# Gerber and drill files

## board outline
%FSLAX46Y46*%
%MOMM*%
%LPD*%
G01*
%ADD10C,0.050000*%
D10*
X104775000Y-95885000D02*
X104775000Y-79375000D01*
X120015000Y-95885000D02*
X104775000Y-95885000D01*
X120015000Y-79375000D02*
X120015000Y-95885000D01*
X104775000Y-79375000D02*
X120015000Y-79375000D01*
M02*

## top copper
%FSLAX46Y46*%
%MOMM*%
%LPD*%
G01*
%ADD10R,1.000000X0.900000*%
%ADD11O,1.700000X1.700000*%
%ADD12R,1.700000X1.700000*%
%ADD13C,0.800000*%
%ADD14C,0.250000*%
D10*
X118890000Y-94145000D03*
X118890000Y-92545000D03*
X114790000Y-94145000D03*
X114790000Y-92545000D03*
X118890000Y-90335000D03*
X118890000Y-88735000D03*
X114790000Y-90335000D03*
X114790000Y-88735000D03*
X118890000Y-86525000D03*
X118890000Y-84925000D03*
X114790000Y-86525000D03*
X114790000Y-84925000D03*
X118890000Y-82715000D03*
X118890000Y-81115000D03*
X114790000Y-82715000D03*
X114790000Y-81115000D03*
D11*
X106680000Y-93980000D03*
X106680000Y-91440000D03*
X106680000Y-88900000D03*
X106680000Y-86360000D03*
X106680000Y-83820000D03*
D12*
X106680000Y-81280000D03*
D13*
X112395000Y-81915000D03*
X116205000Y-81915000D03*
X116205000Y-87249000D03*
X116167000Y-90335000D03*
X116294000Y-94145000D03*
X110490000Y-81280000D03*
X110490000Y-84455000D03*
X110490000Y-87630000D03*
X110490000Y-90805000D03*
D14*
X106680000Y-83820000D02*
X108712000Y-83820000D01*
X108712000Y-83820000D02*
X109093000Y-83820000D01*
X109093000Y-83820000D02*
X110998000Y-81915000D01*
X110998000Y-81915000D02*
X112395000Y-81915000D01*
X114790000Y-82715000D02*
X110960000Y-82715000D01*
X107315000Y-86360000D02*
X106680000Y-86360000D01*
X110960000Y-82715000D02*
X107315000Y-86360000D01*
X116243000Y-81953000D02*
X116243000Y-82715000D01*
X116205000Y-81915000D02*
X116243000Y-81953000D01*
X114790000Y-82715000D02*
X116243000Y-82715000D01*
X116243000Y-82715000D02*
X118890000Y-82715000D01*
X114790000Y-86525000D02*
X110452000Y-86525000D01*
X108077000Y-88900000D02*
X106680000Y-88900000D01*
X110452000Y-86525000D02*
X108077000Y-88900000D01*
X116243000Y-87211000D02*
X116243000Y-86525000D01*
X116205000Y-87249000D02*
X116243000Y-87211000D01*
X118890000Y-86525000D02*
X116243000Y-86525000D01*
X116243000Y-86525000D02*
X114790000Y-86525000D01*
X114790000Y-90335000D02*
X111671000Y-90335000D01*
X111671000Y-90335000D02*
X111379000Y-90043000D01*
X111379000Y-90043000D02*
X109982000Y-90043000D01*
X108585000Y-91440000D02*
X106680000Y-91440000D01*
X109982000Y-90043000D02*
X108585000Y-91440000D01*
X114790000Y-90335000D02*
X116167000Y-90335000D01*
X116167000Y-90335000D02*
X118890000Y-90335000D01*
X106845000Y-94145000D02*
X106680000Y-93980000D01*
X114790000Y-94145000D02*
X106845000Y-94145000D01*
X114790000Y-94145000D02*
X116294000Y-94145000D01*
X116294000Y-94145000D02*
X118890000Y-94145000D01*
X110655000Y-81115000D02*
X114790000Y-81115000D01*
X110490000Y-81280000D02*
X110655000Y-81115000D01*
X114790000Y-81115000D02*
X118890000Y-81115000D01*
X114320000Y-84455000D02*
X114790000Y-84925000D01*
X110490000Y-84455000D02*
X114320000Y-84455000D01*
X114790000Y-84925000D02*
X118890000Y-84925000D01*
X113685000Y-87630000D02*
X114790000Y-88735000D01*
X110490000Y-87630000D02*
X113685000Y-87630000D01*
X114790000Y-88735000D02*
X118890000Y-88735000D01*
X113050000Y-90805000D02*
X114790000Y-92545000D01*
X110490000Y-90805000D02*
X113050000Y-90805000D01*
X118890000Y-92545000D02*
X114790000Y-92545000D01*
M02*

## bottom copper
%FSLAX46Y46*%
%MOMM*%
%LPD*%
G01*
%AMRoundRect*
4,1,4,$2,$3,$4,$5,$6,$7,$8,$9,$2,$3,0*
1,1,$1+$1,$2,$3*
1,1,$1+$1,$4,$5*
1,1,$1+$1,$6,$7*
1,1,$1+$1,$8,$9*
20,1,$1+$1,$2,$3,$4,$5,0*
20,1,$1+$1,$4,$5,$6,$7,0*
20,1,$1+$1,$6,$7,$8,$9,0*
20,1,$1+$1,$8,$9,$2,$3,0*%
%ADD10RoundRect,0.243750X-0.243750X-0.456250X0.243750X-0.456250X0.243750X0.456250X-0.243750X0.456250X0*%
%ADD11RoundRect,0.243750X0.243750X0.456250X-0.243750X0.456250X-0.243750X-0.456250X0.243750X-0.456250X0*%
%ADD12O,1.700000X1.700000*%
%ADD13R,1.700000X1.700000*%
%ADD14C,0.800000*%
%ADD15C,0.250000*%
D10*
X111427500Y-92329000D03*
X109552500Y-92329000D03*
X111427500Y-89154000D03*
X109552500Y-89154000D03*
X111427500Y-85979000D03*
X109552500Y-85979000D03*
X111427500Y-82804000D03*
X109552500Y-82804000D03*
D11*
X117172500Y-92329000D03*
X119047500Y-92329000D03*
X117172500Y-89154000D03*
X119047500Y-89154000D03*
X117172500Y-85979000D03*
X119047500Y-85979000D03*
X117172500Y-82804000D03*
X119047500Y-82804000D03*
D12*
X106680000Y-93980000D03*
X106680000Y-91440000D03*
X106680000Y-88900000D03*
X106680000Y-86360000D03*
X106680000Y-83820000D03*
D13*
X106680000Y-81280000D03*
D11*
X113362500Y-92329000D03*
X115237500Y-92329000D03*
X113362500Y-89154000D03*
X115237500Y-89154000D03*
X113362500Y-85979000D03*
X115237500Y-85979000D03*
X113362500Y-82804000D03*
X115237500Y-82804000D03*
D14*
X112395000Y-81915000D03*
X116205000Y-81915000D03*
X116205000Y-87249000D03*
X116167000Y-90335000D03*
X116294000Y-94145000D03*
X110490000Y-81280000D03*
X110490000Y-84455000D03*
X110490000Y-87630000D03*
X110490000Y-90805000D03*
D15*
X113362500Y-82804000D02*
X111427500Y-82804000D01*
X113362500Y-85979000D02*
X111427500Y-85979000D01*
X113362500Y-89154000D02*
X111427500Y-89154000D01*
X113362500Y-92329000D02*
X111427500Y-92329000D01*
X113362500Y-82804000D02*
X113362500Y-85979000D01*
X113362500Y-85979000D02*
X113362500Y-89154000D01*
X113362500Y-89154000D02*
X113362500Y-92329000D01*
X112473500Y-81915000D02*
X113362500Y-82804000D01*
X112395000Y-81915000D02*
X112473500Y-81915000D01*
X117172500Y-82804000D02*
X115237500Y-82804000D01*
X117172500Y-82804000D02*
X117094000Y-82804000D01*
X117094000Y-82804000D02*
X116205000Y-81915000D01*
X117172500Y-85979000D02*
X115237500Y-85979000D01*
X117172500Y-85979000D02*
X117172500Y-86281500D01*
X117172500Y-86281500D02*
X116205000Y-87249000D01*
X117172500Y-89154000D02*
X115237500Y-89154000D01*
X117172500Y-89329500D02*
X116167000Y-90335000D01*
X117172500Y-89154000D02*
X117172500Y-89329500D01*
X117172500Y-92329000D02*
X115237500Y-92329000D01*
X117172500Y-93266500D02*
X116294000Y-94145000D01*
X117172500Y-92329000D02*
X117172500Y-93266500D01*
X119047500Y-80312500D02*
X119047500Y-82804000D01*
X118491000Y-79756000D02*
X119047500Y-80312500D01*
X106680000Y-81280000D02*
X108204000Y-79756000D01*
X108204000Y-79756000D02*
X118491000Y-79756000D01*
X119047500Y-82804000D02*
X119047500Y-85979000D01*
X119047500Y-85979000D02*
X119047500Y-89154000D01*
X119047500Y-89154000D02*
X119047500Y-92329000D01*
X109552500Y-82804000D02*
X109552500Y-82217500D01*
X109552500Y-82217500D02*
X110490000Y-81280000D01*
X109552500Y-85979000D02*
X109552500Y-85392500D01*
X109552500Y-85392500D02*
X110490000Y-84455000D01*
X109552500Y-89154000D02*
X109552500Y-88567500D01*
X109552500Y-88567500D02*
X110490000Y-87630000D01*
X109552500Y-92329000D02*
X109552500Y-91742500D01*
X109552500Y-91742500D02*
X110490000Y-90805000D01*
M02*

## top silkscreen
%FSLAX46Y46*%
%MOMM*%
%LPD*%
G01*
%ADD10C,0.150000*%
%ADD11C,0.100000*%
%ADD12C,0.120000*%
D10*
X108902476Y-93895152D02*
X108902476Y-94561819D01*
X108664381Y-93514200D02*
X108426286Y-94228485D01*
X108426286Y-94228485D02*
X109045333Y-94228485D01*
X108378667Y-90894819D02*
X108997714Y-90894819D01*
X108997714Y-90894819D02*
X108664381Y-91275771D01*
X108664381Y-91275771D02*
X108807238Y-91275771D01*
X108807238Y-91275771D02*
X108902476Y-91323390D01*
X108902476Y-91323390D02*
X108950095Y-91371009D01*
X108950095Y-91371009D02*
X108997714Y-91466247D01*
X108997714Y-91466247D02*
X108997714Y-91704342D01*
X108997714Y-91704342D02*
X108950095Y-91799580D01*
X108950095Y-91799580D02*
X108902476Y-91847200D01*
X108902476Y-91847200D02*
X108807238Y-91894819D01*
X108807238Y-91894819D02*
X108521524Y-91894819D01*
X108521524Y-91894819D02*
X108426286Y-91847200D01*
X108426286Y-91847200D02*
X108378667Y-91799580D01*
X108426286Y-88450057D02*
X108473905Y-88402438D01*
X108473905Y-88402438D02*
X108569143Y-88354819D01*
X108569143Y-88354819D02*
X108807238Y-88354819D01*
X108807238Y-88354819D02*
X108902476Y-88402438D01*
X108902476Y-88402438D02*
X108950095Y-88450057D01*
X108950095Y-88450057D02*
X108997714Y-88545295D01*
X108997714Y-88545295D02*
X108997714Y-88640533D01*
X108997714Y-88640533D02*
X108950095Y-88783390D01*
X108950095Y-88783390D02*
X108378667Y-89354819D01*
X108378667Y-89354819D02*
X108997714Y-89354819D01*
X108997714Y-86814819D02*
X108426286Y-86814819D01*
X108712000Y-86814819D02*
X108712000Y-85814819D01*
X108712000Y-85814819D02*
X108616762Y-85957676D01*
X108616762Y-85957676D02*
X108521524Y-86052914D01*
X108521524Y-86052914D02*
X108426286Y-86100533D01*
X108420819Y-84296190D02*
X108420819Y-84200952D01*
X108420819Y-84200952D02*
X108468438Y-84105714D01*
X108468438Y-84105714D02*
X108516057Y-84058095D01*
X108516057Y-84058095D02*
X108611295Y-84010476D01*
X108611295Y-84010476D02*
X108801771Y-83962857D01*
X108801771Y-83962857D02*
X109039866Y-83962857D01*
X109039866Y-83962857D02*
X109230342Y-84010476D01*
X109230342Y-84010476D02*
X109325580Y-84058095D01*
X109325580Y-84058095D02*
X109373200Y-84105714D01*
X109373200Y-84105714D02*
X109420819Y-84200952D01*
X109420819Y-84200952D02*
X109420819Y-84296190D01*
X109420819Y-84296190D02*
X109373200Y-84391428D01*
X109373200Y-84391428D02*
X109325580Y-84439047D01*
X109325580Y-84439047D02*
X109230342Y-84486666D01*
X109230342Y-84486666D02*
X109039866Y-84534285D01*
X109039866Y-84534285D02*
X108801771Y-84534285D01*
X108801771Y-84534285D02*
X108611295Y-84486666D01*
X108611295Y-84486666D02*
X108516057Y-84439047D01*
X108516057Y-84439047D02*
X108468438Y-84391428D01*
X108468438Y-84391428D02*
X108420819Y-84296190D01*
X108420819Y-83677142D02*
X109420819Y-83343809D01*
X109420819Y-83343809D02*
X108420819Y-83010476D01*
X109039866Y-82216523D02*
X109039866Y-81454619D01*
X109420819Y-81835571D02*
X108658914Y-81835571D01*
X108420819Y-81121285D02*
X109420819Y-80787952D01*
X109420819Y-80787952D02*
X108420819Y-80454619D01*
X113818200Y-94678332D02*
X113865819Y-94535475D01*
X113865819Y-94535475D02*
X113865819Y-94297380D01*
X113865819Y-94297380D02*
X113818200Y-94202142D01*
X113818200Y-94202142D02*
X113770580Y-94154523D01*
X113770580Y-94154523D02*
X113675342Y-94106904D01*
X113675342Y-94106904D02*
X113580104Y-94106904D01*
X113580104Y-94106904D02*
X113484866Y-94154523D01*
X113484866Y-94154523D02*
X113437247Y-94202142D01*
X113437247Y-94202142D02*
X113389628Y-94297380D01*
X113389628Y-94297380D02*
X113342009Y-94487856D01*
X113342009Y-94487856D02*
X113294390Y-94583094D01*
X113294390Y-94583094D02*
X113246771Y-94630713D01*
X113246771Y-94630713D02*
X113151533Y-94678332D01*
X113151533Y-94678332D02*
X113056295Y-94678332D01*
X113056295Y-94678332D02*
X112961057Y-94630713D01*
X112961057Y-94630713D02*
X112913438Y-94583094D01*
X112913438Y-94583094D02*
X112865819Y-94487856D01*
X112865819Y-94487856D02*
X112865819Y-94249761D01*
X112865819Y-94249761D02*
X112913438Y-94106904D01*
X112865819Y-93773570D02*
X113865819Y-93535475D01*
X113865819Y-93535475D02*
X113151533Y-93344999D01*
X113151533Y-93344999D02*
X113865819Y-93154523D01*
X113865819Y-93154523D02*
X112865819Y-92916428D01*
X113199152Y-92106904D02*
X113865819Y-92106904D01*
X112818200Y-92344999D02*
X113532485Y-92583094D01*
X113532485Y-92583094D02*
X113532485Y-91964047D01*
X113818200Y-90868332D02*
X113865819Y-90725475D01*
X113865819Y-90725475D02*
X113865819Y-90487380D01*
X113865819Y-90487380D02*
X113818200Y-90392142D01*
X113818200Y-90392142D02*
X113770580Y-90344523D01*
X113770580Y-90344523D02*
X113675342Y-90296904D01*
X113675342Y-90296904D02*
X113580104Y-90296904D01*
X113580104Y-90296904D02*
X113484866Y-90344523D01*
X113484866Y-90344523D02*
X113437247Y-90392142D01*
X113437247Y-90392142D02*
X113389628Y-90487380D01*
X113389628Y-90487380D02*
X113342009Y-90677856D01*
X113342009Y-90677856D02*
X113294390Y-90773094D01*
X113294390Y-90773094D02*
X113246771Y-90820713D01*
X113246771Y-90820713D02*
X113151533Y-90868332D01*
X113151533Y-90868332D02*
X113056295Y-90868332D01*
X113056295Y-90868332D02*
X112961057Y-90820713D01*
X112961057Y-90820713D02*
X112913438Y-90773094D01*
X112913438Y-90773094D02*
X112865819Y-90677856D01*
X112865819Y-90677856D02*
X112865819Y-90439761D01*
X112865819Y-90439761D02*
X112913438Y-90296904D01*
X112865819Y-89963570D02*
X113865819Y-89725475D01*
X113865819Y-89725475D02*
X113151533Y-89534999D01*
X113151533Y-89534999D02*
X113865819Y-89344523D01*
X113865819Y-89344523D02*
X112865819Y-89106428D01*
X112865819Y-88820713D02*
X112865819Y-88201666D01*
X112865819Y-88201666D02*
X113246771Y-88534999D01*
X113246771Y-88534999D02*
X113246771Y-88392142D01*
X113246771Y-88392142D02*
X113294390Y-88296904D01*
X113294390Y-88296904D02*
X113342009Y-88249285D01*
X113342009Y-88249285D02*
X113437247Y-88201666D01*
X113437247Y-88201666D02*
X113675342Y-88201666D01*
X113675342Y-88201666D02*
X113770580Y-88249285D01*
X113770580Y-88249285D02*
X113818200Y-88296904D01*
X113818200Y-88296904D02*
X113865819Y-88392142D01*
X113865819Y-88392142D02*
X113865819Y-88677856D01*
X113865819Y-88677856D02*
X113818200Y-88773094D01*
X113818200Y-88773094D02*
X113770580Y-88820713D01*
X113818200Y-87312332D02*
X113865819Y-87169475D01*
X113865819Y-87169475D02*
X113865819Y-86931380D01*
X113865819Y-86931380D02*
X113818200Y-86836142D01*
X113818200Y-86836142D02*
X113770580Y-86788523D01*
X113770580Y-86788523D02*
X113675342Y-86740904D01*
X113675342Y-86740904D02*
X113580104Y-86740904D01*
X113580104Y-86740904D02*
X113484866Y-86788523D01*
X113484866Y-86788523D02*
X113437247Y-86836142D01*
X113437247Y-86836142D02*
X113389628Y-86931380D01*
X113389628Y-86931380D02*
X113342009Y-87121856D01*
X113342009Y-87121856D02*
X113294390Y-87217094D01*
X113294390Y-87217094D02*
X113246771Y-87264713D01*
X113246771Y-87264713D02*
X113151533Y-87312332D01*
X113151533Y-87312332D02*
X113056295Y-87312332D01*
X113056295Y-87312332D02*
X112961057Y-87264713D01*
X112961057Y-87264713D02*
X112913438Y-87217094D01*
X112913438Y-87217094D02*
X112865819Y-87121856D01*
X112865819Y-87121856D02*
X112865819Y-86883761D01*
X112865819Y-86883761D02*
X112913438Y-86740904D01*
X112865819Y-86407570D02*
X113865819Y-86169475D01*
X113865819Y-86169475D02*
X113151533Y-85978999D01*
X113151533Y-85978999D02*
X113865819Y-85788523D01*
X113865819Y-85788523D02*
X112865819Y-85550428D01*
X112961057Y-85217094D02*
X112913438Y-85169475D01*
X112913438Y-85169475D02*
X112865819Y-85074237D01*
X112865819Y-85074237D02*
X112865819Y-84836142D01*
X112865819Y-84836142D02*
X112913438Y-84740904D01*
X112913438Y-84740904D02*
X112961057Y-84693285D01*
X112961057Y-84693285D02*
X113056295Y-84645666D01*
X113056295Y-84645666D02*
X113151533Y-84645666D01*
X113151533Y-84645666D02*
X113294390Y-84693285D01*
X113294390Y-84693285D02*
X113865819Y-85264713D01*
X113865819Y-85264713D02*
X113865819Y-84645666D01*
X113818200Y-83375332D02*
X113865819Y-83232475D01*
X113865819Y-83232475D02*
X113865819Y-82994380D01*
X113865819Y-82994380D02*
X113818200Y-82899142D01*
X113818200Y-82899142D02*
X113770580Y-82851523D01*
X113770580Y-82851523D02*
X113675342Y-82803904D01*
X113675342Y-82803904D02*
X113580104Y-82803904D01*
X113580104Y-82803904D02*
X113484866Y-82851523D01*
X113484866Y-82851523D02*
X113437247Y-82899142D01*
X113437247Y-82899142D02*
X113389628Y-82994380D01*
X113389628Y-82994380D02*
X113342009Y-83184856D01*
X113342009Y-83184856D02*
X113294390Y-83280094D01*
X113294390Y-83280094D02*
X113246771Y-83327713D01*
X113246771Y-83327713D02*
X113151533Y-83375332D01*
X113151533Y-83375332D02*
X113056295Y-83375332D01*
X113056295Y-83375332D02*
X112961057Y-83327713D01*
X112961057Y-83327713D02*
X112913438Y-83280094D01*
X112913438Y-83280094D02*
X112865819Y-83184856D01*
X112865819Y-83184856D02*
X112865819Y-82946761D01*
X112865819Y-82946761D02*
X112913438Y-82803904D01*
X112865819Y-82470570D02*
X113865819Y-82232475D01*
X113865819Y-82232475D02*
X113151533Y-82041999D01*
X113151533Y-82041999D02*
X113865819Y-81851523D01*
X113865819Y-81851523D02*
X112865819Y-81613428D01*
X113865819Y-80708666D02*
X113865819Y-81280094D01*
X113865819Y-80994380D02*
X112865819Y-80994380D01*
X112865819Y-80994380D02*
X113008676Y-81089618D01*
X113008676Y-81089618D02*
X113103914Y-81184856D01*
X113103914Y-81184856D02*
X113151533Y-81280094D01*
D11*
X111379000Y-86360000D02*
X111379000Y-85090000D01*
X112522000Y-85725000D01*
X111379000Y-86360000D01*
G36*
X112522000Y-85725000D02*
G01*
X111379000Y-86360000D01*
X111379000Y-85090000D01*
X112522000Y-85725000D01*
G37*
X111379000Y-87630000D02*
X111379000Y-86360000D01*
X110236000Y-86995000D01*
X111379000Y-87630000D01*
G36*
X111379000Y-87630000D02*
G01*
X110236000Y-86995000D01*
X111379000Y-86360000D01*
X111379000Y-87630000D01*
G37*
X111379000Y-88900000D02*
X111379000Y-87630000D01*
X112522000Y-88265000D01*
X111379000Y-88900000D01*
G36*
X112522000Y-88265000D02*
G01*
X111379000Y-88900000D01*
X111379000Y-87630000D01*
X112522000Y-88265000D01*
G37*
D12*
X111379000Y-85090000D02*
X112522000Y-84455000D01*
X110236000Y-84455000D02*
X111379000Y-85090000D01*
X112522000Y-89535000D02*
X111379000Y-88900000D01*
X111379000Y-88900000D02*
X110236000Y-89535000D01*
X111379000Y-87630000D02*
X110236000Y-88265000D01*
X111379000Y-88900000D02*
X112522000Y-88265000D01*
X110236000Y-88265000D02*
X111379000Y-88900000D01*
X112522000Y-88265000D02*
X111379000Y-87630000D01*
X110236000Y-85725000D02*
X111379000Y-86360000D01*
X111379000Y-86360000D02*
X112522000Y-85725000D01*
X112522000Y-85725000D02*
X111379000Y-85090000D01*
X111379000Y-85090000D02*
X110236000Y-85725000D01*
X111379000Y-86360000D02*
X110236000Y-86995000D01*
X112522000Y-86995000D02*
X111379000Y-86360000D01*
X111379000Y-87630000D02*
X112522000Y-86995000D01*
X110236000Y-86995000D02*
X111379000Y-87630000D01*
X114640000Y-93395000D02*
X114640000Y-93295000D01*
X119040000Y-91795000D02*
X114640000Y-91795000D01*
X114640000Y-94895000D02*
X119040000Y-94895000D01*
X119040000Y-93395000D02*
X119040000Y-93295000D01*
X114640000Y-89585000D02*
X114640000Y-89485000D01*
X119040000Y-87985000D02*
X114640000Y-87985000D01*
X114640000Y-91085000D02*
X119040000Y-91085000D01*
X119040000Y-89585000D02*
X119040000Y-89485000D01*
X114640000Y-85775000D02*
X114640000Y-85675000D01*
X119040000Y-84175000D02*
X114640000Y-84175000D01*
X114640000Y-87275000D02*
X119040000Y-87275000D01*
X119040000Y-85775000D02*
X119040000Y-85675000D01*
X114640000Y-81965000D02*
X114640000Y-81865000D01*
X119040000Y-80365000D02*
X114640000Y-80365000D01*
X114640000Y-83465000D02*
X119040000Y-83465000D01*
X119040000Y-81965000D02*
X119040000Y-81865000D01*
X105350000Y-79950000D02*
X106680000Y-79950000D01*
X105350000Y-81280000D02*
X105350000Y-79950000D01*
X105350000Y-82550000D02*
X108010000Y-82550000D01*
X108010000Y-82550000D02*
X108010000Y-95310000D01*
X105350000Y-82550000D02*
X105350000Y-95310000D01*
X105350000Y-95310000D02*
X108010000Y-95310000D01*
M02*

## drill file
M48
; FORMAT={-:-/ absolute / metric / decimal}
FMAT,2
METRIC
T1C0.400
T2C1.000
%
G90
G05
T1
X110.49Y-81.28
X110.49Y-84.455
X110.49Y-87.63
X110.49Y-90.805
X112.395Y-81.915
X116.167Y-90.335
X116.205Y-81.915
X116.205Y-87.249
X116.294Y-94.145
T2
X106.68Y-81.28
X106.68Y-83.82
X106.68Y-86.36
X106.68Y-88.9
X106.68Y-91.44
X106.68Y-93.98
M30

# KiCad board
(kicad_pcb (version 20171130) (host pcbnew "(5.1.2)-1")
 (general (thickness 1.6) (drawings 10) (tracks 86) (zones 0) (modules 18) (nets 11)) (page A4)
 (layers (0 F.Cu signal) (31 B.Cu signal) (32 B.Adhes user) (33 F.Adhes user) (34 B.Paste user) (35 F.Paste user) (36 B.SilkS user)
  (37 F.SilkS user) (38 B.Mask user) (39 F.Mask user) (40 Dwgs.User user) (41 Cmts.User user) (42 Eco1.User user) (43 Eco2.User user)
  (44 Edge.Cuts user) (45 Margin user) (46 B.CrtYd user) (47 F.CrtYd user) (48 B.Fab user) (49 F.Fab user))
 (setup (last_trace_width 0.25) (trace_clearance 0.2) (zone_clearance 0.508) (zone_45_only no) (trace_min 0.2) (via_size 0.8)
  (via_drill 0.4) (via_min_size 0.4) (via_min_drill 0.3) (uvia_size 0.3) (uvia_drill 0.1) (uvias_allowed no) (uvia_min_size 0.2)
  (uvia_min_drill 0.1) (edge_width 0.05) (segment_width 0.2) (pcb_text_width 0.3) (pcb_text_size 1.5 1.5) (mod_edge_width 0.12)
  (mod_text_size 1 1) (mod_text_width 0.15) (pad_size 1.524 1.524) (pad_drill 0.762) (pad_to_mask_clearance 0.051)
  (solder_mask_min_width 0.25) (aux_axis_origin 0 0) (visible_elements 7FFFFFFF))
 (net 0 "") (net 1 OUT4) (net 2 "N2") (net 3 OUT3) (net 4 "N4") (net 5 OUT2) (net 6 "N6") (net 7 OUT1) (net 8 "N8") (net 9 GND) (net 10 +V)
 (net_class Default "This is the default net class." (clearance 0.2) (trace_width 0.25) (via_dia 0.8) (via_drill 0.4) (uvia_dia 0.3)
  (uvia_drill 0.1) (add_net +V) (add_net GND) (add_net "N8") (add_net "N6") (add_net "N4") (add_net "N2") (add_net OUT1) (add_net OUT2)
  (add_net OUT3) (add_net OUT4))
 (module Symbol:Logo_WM (layer F.Cu) (at 111.379 86.995 90)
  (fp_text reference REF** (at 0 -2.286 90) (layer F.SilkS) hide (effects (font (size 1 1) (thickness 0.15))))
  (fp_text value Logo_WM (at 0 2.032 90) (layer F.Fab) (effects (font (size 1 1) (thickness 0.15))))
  (fp_poly (pts (xy 0.635 0) (xy 1.905 0) (xy 1.27 1.143)) (layer F.SilkS) (width 0.1))
  (fp_poly (pts (xy -0.635 0) (xy 0.635 0) (xy 0 -1.143)) (layer F.SilkS) (width 0.1))
  (fp_poly (pts (xy -1.905 0) (xy -0.635 0) (xy -1.27 1.143)) (layer F.SilkS) (width 0.1))
  (fp_line (start 1.905 0) (end 2.54 1.143) (layer F.SilkS) (width 0.12))
  (fp_line (start 2.54 -1.143) (end 1.905 0) (layer F.SilkS) (width 0.12))
  (fp_line (start -2.54 1.143) (end -1.905 0) (layer F.SilkS) (width 0.12))
  (fp_line (start -1.905 0) (end -2.54 -1.143) (layer F.SilkS) (width 0.12))
  (fp_line (start -0.635 0) (end -1.27 -1.143) (layer F.SilkS) (width 0.12))
  (fp_line (start -1.905 0) (end -1.27 1.143) (layer F.SilkS) (width 0.12))
  (fp_line (start -1.27 -1.143) (end -1.905 0) (layer F.SilkS) (width 0.12))
  (fp_line (start -1.27 1.143) (end -0.635 0) (layer F.SilkS) (width 0.12))
  (fp_line (start 1.27 -1.143) (end 0.635 0) (layer F.SilkS) (width 0.12))
  (fp_line (start 0.635 0) (end 1.27 1.143) (layer F.SilkS) (width 0.12))
  (fp_line (start 1.27 1.143) (end 1.905 0) (layer F.SilkS) (width 0.12))
  (fp_line (start 1.905 0) (end 1.27 -1.143) (layer F.SilkS) (width 0.12))
  (fp_line (start 0.635 0) (end 0 -1.143) (layer F.SilkS) (width 0.12))
  (fp_line (start 0 1.143) (end 0.635 0) (layer F.SilkS) (width 0.12))
  (fp_line (start -0.635 0) (end 0 1.143) (layer F.SilkS) (width 0.12))
  (fp_line (start 0 -1.143) (end -0.635 0) (layer F.SilkS) (width 0.12)))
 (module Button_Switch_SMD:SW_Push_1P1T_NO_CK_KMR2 (layer F.Cu) (at 116.84 93.345)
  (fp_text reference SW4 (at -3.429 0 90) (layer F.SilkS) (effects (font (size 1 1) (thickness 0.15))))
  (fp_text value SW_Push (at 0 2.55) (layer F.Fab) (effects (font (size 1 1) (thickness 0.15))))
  (fp_line (start -2.2 0.05) (end -2.2 -0.05) (layer F.SilkS) (width 0.12))
  (fp_line (start 2.2 -1.55) (end -2.2 -1.55) (layer F.SilkS) (width 0.12))
  (fp_line (start -2.2 1.55) (end 2.2 1.55) (layer F.SilkS) (width 0.12))
  (fp_line (start 2.2 0.05) (end 2.2 -0.05) (layer F.SilkS) (width 0.12))
  (pad 2 smd rect (at 2.05 0.8 90) (size 0.9 1) (layers F.Cu F.Paste F.Mask) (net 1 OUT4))
  (pad 1 smd rect (at 2.05 -0.8 90) (size 0.9 1) (layers F.Cu F.Paste F.Mask) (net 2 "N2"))
  (pad 2 smd rect (at -2.05 0.8 90) (size 0.9 1) (layers F.Cu F.Paste F.Mask) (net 1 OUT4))
  (pad 1 smd rect (at -2.05 -0.8 90) (size 0.9 1) (layers F.Cu F.Paste F.Mask) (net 2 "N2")))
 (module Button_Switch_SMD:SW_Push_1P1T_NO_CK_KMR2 (layer F.Cu) (at 116.84 89.535)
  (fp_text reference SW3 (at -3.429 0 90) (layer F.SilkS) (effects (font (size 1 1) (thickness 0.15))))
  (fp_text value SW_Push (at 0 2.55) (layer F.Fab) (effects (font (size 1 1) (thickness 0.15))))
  (fp_line (start -2.2 0.05) (end -2.2 -0.05) (layer F.SilkS) (width 0.12))
  (fp_line (start 2.2 -1.55) (end -2.2 -1.55) (layer F.SilkS) (width 0.12))
  (fp_line (start -2.2 1.55) (end 2.2 1.55) (layer F.SilkS) (width 0.12))
  (fp_line (start 2.2 0.05) (end 2.2 -0.05) (layer F.SilkS) (width 0.12))
  (pad 2 smd rect (at 2.05 0.8 90) (size 0.9 1) (layers F.Cu F.Paste F.Mask) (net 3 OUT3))
  (pad 1 smd rect (at 2.05 -0.8 90) (size 0.9 1) (layers F.Cu F.Paste F.Mask) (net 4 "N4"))
  (pad 2 smd rect (at -2.05 0.8 90) (size 0.9 1) (layers F.Cu F.Paste F.Mask) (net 3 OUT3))
  (pad 1 smd rect (at -2.05 -0.8 90) (size 0.9 1) (layers F.Cu F.Paste F.Mask) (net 4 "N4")))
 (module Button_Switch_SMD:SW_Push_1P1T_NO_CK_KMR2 (layer F.Cu) (at 116.84 85.725)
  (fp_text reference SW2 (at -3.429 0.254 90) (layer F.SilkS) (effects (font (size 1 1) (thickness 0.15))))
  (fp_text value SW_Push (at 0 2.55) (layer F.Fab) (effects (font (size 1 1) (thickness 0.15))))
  (fp_line (start -2.2 0.05) (end -2.2 -0.05) (layer F.SilkS) (width 0.12))
  (fp_line (start 2.2 -1.55) (end -2.2 -1.55) (layer F.SilkS) (width 0.12))
  (fp_line (start -2.2 1.55) (end 2.2 1.55) (layer F.SilkS) (width 0.12))
  (fp_line (start 2.2 0.05) (end 2.2 -0.05) (layer F.SilkS) (width 0.12))
  (pad 2 smd rect (at 2.05 0.8 90) (size 0.9 1) (layers F.Cu F.Paste F.Mask) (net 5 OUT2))
  (pad 1 smd rect (at 2.05 -0.8 90) (size 0.9 1) (layers F.Cu F.Paste F.Mask) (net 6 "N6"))
  (pad 2 smd rect (at -2.05 0.8 90) (size 0.9 1) (layers F.Cu F.Paste F.Mask) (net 5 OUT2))
  (pad 1 smd rect (at -2.05 -0.8 90) (size 0.9 1) (layers F.Cu F.Paste F.Mask) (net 6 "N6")))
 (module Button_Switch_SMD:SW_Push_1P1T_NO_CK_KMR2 (layer F.Cu) (at 116.84 81.915)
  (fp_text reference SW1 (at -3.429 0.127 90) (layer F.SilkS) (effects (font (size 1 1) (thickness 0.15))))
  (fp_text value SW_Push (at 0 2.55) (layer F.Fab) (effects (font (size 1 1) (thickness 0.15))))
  (fp_line (start -2.2 0.05) (end -2.2 -0.05) (layer F.SilkS) (width 0.12))
  (fp_line (start 2.2 -1.55) (end -2.2 -1.55) (layer F.SilkS) (width 0.12))
  (fp_line (start -2.2 1.55) (end 2.2 1.55) (layer F.SilkS) (width 0.12))
  (fp_line (start 2.2 0.05) (end 2.2 -0.05) (layer F.SilkS) (width 0.12))
  (pad 2 smd rect (at 2.05 0.8 90) (size 0.9 1) (layers F.Cu F.Paste F.Mask) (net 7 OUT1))
  (pad 1 smd rect (at 2.05 -0.8 90) (size 0.9 1) (layers F.Cu F.Paste F.Mask) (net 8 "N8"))
  (pad 2 smd rect (at -2.05 0.8 90) (size 0.9 1) (layers F.Cu F.Paste F.Mask) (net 7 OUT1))
  (pad 1 smd rect (at -2.05 -0.8 90) (size 0.9 1) (layers F.Cu F.Paste F.Mask) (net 8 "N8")))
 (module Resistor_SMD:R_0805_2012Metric (layer B.Cu) (at 110.49 92.329)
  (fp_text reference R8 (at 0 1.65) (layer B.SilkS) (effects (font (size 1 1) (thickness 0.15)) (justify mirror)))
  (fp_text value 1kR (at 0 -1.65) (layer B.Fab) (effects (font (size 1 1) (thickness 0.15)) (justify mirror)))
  (pad 2 smd roundrect (at 0.9375 0) (size 0.975 1.4) (layers B.Cu B.Paste B.Mask) (roundrect_rratio 0.25) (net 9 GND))
  (pad 1 smd roundrect (at -0.9375 0) (size 0.975 1.4) (layers B.Cu B.Paste B.Mask) (roundrect_rratio 0.25) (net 2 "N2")))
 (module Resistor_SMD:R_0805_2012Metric (layer B.Cu) (at 110.49 89.154)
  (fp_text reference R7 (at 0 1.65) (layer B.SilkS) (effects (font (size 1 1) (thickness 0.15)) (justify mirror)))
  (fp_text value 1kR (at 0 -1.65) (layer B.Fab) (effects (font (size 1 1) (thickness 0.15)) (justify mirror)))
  (pad 2 smd roundrect (at 0.9375 0) (size 0.975 1.4) (layers B.Cu B.Paste B.Mask) (roundrect_rratio 0.25) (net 9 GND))
  (pad 1 smd roundrect (at -0.9375 0) (size 0.975 1.4) (layers B.Cu B.Paste B.Mask) (roundrect_rratio 0.25) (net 4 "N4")))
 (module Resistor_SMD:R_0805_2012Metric (layer B.Cu) (at 110.49 85.979)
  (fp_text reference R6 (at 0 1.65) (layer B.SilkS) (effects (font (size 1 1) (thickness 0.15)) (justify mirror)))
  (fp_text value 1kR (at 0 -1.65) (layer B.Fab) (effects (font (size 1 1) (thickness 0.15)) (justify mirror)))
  (pad 2 smd roundrect (at 0.9375 0) (size 0.975 1.4) (layers B.Cu B.Paste B.Mask) (roundrect_rratio 0.25) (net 9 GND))
  (pad 1 smd roundrect (at -0.9375 0) (size 0.975 1.4) (layers B.Cu B.Paste B.Mask) (roundrect_rratio 0.25) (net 6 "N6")))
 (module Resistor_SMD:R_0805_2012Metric (layer B.Cu) (at 110.49 82.804)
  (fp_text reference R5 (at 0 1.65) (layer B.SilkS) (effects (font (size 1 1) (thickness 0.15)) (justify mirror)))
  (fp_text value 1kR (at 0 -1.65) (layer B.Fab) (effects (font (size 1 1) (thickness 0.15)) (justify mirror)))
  (pad 2 smd roundrect (at 0.9375 0) (size 0.975 1.4) (layers B.Cu B.Paste B.Mask) (roundrect_rratio 0.25) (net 9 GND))
  (pad 1 smd roundrect (at -0.9375 0) (size 0.975 1.4) (layers B.Cu B.Paste B.Mask) (roundrect_rratio 0.25) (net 8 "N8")))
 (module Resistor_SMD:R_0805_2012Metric (layer B.Cu) (at 118.11 92.329 180)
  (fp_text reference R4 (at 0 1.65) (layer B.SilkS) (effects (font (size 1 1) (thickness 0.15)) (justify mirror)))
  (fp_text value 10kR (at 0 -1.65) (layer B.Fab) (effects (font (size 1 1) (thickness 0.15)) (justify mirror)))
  (pad 2 smd roundrect (at 0.9375 0 180) (size 0.975 1.4) (layers B.Cu B.Paste B.Mask) (roundrect_rratio 0.25) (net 1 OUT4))
  (pad 1 smd roundrect (at -0.9375 0 180) (size 0.975 1.4) (layers B.Cu B.Paste B.Mask) (roundrect_rratio 0.25) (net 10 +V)))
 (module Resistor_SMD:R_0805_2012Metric (layer B.Cu) (at 118.11 89.154 180)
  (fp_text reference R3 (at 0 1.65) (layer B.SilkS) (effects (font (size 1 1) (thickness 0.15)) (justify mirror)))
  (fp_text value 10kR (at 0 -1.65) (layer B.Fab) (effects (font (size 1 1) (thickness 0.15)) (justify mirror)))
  (pad 2 smd roundrect (at 0.9375 0 180) (size 0.975 1.4) (layers B.Cu B.Paste B.Mask) (roundrect_rratio 0.25) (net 3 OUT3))
  (pad 1 smd roundrect (at -0.9375 0 180) (size 0.975 1.4) (layers B.Cu B.Paste B.Mask) (roundrect_rratio 0.25) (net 10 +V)))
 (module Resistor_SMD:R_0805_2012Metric (layer B.Cu) (at 118.11 85.979 180)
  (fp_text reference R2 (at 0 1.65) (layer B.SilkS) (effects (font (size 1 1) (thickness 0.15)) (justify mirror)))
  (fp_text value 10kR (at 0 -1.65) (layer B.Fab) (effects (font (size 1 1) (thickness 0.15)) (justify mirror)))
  (pad 2 smd roundrect (at 0.9375 0 180) (size 0.975 1.4) (layers B.Cu B.Paste B.Mask) (roundrect_rratio 0.25) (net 5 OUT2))
  (pad 1 smd roundrect (at -0.9375 0 180) (size 0.975 1.4) (layers B.Cu B.Paste B.Mask) (roundrect_rratio 0.25) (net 10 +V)))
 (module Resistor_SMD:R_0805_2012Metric (layer B.Cu) (at 118.11 82.804 180)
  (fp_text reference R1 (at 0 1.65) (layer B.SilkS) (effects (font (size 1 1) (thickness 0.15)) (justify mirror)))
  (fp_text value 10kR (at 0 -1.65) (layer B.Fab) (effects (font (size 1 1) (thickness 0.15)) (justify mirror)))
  (pad 2 smd roundrect (at 0.9375 0 180) (size 0.975 1.4) (layers B.Cu B.Paste B.Mask) (roundrect_rratio 0.25) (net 7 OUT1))
  (pad 1 smd roundrect (at -0.9375 0 180) (size 0.975 1.4) (layers B.Cu B.Paste B.Mask) (roundrect_rratio 0.25) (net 10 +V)))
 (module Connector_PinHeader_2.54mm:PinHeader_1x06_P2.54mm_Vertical (layer F.Cu) (at 106.68 81.28)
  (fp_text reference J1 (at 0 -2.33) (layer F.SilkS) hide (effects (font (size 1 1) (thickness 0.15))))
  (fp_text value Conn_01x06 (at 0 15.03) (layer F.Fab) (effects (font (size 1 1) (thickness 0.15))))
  (fp_line (start -1.33 -1.33) (end 0 -1.33) (layer F.SilkS) (width 0.12))
  (fp_line (start -1.33 0) (end -1.33 -1.33) (layer F.SilkS) (width 0.12))
  (fp_line (start -1.33 1.27) (end 1.33 1.27) (layer F.SilkS) (width 0.12))
  (fp_line (start 1.33 1.27) (end 1.33 14.03) (layer F.SilkS) (width 0.12))
  (fp_line (start -1.33 1.27) (end -1.33 14.03) (layer F.SilkS) (width 0.12))
  (fp_line (start -1.33 14.03) (end 1.33 14.03) (layer F.SilkS) (width 0.12))
  (pad 6 thru_hole oval (at 0 12.7) (size 1.7 1.7) (drill 1) (layers *.Cu *.Mask) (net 1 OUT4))
  (pad 5 thru_hole oval (at 0 10.16) (size 1.7 1.7) (drill 1) (layers *.Cu *.Mask) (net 3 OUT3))
  (pad 4 thru_hole oval (at 0 7.62) (size 1.7 1.7) (drill 1) (layers *.Cu *.Mask) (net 5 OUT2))
  (pad 3 thru_hole oval (at 0 5.08) (size 1.7 1.7) (drill 1) (layers *.Cu *.Mask) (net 7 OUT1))
  (pad 2 thru_hole oval (at 0 2.54) (size 1.7 1.7) (drill 1) (layers *.Cu *.Mask) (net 9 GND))
  (pad 1 thru_hole rect (at 0 0) (size 1.7 1.7) (drill 1) (layers *.Cu *.Mask) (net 10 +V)))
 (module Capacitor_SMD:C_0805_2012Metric (layer B.Cu) (at 114.3 92.329 180)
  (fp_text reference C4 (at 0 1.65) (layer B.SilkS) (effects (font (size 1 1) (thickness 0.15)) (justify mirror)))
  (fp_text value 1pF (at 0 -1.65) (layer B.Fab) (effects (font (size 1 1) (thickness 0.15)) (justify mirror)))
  (pad 2 smd roundrect (at 0.9375 0 180) (size 0.975 1.4) (layers B.Cu B.Paste B.Mask) (roundrect_rratio 0.25) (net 9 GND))
  (pad 1 smd roundrect (at -0.9375 0 180) (size 0.975 1.4) (layers B.Cu B.Paste B.Mask) (roundrect_rratio 0.25) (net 1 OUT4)))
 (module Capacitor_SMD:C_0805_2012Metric (layer B.Cu) (at 114.3 89.154 180)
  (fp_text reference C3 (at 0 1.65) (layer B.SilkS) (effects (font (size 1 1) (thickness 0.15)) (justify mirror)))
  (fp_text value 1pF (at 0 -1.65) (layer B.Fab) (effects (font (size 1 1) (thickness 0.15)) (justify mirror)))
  (pad 2 smd roundrect (at 0.9375 0 180) (size 0.975 1.4) (layers B.Cu B.Paste B.Mask) (roundrect_rratio 0.25) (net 9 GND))
  (pad 1 smd roundrect (at -0.9375 0 180) (size 0.975 1.4) (layers B.Cu B.Paste B.Mask) (roundrect_rratio 0.25) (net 3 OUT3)))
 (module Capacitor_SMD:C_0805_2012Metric (layer B.Cu) (at 114.3 85.979 180)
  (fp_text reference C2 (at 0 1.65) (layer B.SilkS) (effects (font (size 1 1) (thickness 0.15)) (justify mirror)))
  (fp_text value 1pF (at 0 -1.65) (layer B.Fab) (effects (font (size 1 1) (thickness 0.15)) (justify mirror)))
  (pad 2 smd roundrect (at 0.9375 0 180) (size 0.975 1.4) (layers B.Cu B.Paste B.Mask) (roundrect_rratio 0.25) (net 9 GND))
  (pad 1 smd roundrect (at -0.9375 0 180) (size 0.975 1.4) (layers B.Cu B.Paste B.Mask) (roundrect_rratio 0.25) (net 5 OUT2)))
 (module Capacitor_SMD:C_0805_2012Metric (layer B.Cu) (at 114.3 82.804 180)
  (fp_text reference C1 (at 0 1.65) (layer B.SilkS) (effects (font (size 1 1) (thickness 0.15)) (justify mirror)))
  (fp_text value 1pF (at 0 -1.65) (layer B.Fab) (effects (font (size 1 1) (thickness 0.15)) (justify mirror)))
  (pad 2 smd roundrect (at 0.9375 0 180) (size 0.975 1.4) (layers B.Cu B.Paste B.Mask) (roundrect_rratio 0.25) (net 9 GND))
  (pad 1 smd roundrect (at -0.9375 0 180) (size 0.975 1.4) (layers B.Cu B.Paste B.Mask) (roundrect_rratio 0.25) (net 7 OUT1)))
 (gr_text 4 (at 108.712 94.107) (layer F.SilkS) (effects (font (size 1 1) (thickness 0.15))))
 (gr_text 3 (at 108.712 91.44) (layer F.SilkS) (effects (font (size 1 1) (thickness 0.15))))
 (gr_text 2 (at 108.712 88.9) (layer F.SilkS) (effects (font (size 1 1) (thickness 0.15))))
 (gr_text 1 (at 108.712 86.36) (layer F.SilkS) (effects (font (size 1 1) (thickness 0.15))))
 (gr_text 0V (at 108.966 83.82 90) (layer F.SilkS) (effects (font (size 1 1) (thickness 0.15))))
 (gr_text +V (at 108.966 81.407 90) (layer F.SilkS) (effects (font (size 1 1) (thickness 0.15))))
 (gr_line (start 104.775 95.885) (end 104.775 79.375) (layer Edge.Cuts) (width 0.05))
 (gr_line (start 120.015 95.885) (end 104.775 95.885) (layer Edge.Cuts) (width 0.05))
 (gr_line (start 120.015 79.375) (end 120.015 95.885) (layer Edge.Cuts) (width 0.05))
 (gr_line (start 104.775 79.375) (end 120.015 79.375) (layer Edge.Cuts) (width 0.05))
 (segment (start 113.3625 82.804) (end 111.4275 82.804) (width 0.25) (layer B.Cu) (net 9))
 (segment (start 113.3625 85.979) (end 111.4275 85.979) (width 0.25) (layer B.Cu) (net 9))
 (segment (start 113.3625 89.154) (end 111.4275 89.154) (width 0.25) (layer B.Cu) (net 9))
 (segment (start 113.3625 92.329) (end 111.4275 92.329) (width 0.25) (layer B.Cu) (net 9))
 (segment (start 113.3625 82.804) (end 113.3625 85.979) (width 0.25) (layer B.Cu) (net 9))
 (segment (start 113.3625 85.979) (end 113.3625 89.154) (width 0.25) (layer B.Cu) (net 9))
 (segment (start 113.3625 89.154) (end 113.3625 92.329) (width 0.25) (layer B.Cu) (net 9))
 (segment (start 106.68 83.82) (end 108.712 83.82) (width 0.25) (layer F.Cu) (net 9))
 (segment (start 108.712 83.82) (end 109.093 83.82) (width 0.25) (layer F.Cu) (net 9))
 (via (at 112.395 81.915) (size 0.8) (drill 0.4) (layers F.Cu B.Cu) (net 9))
 (segment (start 109.093 83.82) (end 110.998 81.915) (width 0.25) (layer F.Cu) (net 9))
 (segment (start 110.998 81.915) (end 112.395 81.915) (width 0.25) (layer F.Cu) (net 9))
 (segment (start 112.4735 81.915) (end 113.3625 82.804) (width 0.25) (layer B.Cu) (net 9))
 (segment (start 112.395 81.915) (end 112.4735 81.915) (width 0.25) (layer B.Cu) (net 9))
 (segment (start 117.1725 82.804) (end 115.2375 82.804) (width 0.25) (layer B.Cu) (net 7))
 (segment (start 114.79 82.715) (end 110.96 82.715) (width 0.25) (layer F.Cu) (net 7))
 (segment (start 107.315 86.36) (end 106.68 86.36) (width 0.25) (layer F.Cu) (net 7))
 (segment (start 110.96 82.715) (end 107.315 86.36) (width 0.25) (layer F.Cu) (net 7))
 (via (at 116.205 81.915) (size 0.8) (drill 0.4) (layers F.Cu B.Cu) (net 7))
 (segment (start 117.1725 82.804) (end 117.094 82.804) (width 0.25) (layer B.Cu) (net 7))
 (segment (start 117.094 82.804) (end 116.205 81.915) (width 0.25) (layer B.Cu) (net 7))
 (segment (start 116.243 81.953) (end 116.243 82.715) (width 0.25) (layer F.Cu) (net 7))
 (segment (start 116.205 81.915) (end 116.243 81.953) (width 0.25) (layer F.Cu) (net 7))
 (segment (start 114.79 82.715) (end 116.243 82.715) (width 0.25) (layer F.Cu) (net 7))
 (segment (start 116.243 82.715) (end 118.89 82.715) (width 0.25) (layer F.Cu) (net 7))
 (segment (start 117.1725 85.979) (end 115.2375 85.979) (width 0.25) (layer B.Cu) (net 5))
 (segment (start 114.79 86.525) (end 110.452 86.525) (width 0.25) (layer F.Cu) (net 5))
 (segment (start 108.077 88.9) (end 106.68 88.9) (width 0.25) (layer F.Cu) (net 5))
 (segment (start 110.452 86.525) (end 108.077 88.9) (width 0.25) (layer F.Cu) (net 5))
 (via (at 116.205 87.249) (size 0.8) (drill 0.4) (layers F.Cu B.Cu) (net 5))
 (segment (start 117.1725 85.979) (end 117.1725 86.2815) (width 0.25) (layer B.Cu) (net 5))
 (segment (start 117.1725 86.2815) (end 116.205 87.249) (width 0.25) (layer B.Cu) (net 5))
 (segment (start 116.243 87.211) (end 116.243 86.525) (width 0.25) (layer F.Cu) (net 5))
 (segment (start 116.205 87.249) (end 116.243 87.211) (width 0.25) (layer F.Cu) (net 5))
 (segment (start 118.89 86.525) (end 116.243 86.525) (width 0.25) (layer F.Cu) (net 5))
 (segment (start 116.243 86.525) (end 114.79 86.525) (width 0.25) (layer F.Cu) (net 5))
 (segment (start 117.1725 89.154) (end 115.2375 89.154) (width 0.25) (layer B.Cu) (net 3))
 (segment (start 114.79 90.335) (end 111.671 90.335) (width 0.25) (layer F.Cu) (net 3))
 (segment (start 111.671 90.335) (end 111.379 90.043) (width 0.25) (layer F.Cu) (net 3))
 (segment (start 111.379 90.043) (end 109.982 90.043) (width 0.25) (layer F.Cu) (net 3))
 (segment (start 108.585 91.44) (end 106.68 91.44) (width 0.25) (layer F.Cu) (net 3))
 (segment (start 109.982 90.043) (end 108.585 91.44) (width 0.25) (layer F.Cu) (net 3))
 (via (at 116.167 90.335) (size 0.8) (drill 0.4) (layers F.Cu B.Cu) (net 3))
 (segment (start 117.1725 89.3295) (end 116.167 90.335) (width 0.25) (layer B.Cu) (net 3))
 (segment (start 117.1725 89.154) (end 117.1725 89.3295) (width 0.25) (layer B.Cu) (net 3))
 (segment (start 114.79 90.335) (end 116.167 90.335) (width 0.25) (layer F.Cu) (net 3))
 (segment (start 116.167 90.335) (end 118.89 90.335) (width 0.25) (layer F.Cu) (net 3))
 (segment (start 117.1725 92.329) (end 115.2375 92.329) (width 0.25) (layer B.Cu) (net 1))
 (segment (start 106.845 94.145) (end 106.68 93.98) (width 0.25) (layer F.Cu) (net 1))
 (segment (start 114.79 94.145) (end 106.845 94.145) (width 0.25) (layer F.Cu) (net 1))
 (via (at 116.294 94.145) (size 0.8) (drill 0.4) (layers F.Cu B.Cu) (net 1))
 (segment (start 117.1725 93.2665) (end 116.294 94.145) (width 0.25) (layer B.Cu) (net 1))
 (segment (start 117.1725 92.329) (end 117.1725 93.2665) (width 0.25) (layer B.Cu) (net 1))
 (segment (start 114.79 94.145) (end 116.294 94.145) (width 0.25) (layer F.Cu) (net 1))
 (segment (start 116.294 94.145) (end 118.89 94.145) (width 0.25) (layer F.Cu) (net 1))
 (segment (start 119.0475 80.3125) (end 119.0475 82.804) (width 0.25) (layer B.Cu) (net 10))
 (segment (start 118.491 79.756) (end 119.0475 80.3125) (width 0.25) (layer B.Cu) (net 10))
 (segment (start 106.68 81.28) (end 108.204 79.756) (width 0.25) (layer B.Cu) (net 10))
 (segment (start 108.204 79.756) (end 118.491 79.756) (width 0.25) (layer B.Cu) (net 10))
 (segment (start 119.0475 82.804) (end 119.0475 85.979) (width 0.25) (layer B.Cu) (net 10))
 (segment (start 119.0475 85.979) (end 119.0475 89.154) (width 0.25) (layer B.Cu) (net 10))
 (segment (start 119.0475 89.154) (end 119.0475 92.329) (width 0.25) (layer B.Cu) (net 10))
 (via (at 110.49 81.28) (size 0.8) (drill 0.4) (layers F.Cu B.Cu) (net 8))
 (segment (start 109.5525 82.804) (end 109.5525 82.2175) (width 0.25) (layer B.Cu) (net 8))
 (segment (start 109.5525 82.2175) (end 110.49 81.28) (width 0.25) (layer B.Cu) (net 8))
 (segment (start 110.655 81.115) (end 114.79 81.115) (width 0.25) (layer F.Cu) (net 8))
 (segment (start 110.49 81.28) (end 110.655 81.115) (width 0.25) (layer F.Cu) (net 8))
 (segment (start 114.79 81.115) (end 118.89 81.115) (width 0.25) (layer F.Cu) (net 8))
 (via (at 110.49 84.455) (size 0.8) (drill 0.4) (layers F.Cu B.Cu) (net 6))
 (segment (start 109.5525 85.979) (end 109.5525 85.3925) (width 0.25) (layer B.Cu) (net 6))
 (segment (start 109.5525 85.3925) (end 110.49 84.455) (width 0.25) (layer B.Cu) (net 6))
 (segment (start 114.32 84.455) (end 114.79 84.925) (width 0.25) (layer F.Cu) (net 6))
 (segment (start 110.49 84.455) (end 114.32 84.455) (width 0.25) (layer F.Cu) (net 6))
 (segment (start 114.79 84.925) (end 118.89 84.925) (width 0.25) (layer F.Cu) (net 6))
 (via (at 110.49 87.63) (size 0.8) (drill 0.4) (layers F.Cu B.Cu) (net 4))
 (segment (start 109.5525 89.154) (end 109.5525 88.5675) (width 0.25) (layer B.Cu) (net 4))
 (segment (start 109.5525 88.5675) (end 110.49 87.63) (width 0.25) (layer B.Cu) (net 4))
 (segment (start 113.685 87.63) (end 114.79 88.735) (width 0.25) (layer F.Cu) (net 4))
 (segment (start 110.49 87.63) (end 113.685 87.63) (width 0.25) (layer F.Cu) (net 4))
 (segment (start 114.79 88.735) (end 118.89 88.735) (width 0.25) (layer F.Cu) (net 4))
 (via (at 110.49 90.805) (size 0.8) (drill 0.4) (layers F.Cu B.Cu) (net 2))
 (segment (start 109.5525 92.329) (end 109.5525 91.7425) (width 0.25) (layer B.Cu) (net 2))
 (segment (start 109.5525 91.7425) (end 110.49 90.805) (width 0.25) (layer B.Cu) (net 2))
 (segment (start 113.05 90.805) (end 114.79 92.545) (width 0.25) (layer F.Cu) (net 2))
 (segment (start 110.49 90.805) (end 113.05 90.805) (width 0.25) (layer F.Cu) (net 2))
 (segment (start 118.89 92.545) (end 114.79 92.545) (width 0.25) (layer F.Cu) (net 2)))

